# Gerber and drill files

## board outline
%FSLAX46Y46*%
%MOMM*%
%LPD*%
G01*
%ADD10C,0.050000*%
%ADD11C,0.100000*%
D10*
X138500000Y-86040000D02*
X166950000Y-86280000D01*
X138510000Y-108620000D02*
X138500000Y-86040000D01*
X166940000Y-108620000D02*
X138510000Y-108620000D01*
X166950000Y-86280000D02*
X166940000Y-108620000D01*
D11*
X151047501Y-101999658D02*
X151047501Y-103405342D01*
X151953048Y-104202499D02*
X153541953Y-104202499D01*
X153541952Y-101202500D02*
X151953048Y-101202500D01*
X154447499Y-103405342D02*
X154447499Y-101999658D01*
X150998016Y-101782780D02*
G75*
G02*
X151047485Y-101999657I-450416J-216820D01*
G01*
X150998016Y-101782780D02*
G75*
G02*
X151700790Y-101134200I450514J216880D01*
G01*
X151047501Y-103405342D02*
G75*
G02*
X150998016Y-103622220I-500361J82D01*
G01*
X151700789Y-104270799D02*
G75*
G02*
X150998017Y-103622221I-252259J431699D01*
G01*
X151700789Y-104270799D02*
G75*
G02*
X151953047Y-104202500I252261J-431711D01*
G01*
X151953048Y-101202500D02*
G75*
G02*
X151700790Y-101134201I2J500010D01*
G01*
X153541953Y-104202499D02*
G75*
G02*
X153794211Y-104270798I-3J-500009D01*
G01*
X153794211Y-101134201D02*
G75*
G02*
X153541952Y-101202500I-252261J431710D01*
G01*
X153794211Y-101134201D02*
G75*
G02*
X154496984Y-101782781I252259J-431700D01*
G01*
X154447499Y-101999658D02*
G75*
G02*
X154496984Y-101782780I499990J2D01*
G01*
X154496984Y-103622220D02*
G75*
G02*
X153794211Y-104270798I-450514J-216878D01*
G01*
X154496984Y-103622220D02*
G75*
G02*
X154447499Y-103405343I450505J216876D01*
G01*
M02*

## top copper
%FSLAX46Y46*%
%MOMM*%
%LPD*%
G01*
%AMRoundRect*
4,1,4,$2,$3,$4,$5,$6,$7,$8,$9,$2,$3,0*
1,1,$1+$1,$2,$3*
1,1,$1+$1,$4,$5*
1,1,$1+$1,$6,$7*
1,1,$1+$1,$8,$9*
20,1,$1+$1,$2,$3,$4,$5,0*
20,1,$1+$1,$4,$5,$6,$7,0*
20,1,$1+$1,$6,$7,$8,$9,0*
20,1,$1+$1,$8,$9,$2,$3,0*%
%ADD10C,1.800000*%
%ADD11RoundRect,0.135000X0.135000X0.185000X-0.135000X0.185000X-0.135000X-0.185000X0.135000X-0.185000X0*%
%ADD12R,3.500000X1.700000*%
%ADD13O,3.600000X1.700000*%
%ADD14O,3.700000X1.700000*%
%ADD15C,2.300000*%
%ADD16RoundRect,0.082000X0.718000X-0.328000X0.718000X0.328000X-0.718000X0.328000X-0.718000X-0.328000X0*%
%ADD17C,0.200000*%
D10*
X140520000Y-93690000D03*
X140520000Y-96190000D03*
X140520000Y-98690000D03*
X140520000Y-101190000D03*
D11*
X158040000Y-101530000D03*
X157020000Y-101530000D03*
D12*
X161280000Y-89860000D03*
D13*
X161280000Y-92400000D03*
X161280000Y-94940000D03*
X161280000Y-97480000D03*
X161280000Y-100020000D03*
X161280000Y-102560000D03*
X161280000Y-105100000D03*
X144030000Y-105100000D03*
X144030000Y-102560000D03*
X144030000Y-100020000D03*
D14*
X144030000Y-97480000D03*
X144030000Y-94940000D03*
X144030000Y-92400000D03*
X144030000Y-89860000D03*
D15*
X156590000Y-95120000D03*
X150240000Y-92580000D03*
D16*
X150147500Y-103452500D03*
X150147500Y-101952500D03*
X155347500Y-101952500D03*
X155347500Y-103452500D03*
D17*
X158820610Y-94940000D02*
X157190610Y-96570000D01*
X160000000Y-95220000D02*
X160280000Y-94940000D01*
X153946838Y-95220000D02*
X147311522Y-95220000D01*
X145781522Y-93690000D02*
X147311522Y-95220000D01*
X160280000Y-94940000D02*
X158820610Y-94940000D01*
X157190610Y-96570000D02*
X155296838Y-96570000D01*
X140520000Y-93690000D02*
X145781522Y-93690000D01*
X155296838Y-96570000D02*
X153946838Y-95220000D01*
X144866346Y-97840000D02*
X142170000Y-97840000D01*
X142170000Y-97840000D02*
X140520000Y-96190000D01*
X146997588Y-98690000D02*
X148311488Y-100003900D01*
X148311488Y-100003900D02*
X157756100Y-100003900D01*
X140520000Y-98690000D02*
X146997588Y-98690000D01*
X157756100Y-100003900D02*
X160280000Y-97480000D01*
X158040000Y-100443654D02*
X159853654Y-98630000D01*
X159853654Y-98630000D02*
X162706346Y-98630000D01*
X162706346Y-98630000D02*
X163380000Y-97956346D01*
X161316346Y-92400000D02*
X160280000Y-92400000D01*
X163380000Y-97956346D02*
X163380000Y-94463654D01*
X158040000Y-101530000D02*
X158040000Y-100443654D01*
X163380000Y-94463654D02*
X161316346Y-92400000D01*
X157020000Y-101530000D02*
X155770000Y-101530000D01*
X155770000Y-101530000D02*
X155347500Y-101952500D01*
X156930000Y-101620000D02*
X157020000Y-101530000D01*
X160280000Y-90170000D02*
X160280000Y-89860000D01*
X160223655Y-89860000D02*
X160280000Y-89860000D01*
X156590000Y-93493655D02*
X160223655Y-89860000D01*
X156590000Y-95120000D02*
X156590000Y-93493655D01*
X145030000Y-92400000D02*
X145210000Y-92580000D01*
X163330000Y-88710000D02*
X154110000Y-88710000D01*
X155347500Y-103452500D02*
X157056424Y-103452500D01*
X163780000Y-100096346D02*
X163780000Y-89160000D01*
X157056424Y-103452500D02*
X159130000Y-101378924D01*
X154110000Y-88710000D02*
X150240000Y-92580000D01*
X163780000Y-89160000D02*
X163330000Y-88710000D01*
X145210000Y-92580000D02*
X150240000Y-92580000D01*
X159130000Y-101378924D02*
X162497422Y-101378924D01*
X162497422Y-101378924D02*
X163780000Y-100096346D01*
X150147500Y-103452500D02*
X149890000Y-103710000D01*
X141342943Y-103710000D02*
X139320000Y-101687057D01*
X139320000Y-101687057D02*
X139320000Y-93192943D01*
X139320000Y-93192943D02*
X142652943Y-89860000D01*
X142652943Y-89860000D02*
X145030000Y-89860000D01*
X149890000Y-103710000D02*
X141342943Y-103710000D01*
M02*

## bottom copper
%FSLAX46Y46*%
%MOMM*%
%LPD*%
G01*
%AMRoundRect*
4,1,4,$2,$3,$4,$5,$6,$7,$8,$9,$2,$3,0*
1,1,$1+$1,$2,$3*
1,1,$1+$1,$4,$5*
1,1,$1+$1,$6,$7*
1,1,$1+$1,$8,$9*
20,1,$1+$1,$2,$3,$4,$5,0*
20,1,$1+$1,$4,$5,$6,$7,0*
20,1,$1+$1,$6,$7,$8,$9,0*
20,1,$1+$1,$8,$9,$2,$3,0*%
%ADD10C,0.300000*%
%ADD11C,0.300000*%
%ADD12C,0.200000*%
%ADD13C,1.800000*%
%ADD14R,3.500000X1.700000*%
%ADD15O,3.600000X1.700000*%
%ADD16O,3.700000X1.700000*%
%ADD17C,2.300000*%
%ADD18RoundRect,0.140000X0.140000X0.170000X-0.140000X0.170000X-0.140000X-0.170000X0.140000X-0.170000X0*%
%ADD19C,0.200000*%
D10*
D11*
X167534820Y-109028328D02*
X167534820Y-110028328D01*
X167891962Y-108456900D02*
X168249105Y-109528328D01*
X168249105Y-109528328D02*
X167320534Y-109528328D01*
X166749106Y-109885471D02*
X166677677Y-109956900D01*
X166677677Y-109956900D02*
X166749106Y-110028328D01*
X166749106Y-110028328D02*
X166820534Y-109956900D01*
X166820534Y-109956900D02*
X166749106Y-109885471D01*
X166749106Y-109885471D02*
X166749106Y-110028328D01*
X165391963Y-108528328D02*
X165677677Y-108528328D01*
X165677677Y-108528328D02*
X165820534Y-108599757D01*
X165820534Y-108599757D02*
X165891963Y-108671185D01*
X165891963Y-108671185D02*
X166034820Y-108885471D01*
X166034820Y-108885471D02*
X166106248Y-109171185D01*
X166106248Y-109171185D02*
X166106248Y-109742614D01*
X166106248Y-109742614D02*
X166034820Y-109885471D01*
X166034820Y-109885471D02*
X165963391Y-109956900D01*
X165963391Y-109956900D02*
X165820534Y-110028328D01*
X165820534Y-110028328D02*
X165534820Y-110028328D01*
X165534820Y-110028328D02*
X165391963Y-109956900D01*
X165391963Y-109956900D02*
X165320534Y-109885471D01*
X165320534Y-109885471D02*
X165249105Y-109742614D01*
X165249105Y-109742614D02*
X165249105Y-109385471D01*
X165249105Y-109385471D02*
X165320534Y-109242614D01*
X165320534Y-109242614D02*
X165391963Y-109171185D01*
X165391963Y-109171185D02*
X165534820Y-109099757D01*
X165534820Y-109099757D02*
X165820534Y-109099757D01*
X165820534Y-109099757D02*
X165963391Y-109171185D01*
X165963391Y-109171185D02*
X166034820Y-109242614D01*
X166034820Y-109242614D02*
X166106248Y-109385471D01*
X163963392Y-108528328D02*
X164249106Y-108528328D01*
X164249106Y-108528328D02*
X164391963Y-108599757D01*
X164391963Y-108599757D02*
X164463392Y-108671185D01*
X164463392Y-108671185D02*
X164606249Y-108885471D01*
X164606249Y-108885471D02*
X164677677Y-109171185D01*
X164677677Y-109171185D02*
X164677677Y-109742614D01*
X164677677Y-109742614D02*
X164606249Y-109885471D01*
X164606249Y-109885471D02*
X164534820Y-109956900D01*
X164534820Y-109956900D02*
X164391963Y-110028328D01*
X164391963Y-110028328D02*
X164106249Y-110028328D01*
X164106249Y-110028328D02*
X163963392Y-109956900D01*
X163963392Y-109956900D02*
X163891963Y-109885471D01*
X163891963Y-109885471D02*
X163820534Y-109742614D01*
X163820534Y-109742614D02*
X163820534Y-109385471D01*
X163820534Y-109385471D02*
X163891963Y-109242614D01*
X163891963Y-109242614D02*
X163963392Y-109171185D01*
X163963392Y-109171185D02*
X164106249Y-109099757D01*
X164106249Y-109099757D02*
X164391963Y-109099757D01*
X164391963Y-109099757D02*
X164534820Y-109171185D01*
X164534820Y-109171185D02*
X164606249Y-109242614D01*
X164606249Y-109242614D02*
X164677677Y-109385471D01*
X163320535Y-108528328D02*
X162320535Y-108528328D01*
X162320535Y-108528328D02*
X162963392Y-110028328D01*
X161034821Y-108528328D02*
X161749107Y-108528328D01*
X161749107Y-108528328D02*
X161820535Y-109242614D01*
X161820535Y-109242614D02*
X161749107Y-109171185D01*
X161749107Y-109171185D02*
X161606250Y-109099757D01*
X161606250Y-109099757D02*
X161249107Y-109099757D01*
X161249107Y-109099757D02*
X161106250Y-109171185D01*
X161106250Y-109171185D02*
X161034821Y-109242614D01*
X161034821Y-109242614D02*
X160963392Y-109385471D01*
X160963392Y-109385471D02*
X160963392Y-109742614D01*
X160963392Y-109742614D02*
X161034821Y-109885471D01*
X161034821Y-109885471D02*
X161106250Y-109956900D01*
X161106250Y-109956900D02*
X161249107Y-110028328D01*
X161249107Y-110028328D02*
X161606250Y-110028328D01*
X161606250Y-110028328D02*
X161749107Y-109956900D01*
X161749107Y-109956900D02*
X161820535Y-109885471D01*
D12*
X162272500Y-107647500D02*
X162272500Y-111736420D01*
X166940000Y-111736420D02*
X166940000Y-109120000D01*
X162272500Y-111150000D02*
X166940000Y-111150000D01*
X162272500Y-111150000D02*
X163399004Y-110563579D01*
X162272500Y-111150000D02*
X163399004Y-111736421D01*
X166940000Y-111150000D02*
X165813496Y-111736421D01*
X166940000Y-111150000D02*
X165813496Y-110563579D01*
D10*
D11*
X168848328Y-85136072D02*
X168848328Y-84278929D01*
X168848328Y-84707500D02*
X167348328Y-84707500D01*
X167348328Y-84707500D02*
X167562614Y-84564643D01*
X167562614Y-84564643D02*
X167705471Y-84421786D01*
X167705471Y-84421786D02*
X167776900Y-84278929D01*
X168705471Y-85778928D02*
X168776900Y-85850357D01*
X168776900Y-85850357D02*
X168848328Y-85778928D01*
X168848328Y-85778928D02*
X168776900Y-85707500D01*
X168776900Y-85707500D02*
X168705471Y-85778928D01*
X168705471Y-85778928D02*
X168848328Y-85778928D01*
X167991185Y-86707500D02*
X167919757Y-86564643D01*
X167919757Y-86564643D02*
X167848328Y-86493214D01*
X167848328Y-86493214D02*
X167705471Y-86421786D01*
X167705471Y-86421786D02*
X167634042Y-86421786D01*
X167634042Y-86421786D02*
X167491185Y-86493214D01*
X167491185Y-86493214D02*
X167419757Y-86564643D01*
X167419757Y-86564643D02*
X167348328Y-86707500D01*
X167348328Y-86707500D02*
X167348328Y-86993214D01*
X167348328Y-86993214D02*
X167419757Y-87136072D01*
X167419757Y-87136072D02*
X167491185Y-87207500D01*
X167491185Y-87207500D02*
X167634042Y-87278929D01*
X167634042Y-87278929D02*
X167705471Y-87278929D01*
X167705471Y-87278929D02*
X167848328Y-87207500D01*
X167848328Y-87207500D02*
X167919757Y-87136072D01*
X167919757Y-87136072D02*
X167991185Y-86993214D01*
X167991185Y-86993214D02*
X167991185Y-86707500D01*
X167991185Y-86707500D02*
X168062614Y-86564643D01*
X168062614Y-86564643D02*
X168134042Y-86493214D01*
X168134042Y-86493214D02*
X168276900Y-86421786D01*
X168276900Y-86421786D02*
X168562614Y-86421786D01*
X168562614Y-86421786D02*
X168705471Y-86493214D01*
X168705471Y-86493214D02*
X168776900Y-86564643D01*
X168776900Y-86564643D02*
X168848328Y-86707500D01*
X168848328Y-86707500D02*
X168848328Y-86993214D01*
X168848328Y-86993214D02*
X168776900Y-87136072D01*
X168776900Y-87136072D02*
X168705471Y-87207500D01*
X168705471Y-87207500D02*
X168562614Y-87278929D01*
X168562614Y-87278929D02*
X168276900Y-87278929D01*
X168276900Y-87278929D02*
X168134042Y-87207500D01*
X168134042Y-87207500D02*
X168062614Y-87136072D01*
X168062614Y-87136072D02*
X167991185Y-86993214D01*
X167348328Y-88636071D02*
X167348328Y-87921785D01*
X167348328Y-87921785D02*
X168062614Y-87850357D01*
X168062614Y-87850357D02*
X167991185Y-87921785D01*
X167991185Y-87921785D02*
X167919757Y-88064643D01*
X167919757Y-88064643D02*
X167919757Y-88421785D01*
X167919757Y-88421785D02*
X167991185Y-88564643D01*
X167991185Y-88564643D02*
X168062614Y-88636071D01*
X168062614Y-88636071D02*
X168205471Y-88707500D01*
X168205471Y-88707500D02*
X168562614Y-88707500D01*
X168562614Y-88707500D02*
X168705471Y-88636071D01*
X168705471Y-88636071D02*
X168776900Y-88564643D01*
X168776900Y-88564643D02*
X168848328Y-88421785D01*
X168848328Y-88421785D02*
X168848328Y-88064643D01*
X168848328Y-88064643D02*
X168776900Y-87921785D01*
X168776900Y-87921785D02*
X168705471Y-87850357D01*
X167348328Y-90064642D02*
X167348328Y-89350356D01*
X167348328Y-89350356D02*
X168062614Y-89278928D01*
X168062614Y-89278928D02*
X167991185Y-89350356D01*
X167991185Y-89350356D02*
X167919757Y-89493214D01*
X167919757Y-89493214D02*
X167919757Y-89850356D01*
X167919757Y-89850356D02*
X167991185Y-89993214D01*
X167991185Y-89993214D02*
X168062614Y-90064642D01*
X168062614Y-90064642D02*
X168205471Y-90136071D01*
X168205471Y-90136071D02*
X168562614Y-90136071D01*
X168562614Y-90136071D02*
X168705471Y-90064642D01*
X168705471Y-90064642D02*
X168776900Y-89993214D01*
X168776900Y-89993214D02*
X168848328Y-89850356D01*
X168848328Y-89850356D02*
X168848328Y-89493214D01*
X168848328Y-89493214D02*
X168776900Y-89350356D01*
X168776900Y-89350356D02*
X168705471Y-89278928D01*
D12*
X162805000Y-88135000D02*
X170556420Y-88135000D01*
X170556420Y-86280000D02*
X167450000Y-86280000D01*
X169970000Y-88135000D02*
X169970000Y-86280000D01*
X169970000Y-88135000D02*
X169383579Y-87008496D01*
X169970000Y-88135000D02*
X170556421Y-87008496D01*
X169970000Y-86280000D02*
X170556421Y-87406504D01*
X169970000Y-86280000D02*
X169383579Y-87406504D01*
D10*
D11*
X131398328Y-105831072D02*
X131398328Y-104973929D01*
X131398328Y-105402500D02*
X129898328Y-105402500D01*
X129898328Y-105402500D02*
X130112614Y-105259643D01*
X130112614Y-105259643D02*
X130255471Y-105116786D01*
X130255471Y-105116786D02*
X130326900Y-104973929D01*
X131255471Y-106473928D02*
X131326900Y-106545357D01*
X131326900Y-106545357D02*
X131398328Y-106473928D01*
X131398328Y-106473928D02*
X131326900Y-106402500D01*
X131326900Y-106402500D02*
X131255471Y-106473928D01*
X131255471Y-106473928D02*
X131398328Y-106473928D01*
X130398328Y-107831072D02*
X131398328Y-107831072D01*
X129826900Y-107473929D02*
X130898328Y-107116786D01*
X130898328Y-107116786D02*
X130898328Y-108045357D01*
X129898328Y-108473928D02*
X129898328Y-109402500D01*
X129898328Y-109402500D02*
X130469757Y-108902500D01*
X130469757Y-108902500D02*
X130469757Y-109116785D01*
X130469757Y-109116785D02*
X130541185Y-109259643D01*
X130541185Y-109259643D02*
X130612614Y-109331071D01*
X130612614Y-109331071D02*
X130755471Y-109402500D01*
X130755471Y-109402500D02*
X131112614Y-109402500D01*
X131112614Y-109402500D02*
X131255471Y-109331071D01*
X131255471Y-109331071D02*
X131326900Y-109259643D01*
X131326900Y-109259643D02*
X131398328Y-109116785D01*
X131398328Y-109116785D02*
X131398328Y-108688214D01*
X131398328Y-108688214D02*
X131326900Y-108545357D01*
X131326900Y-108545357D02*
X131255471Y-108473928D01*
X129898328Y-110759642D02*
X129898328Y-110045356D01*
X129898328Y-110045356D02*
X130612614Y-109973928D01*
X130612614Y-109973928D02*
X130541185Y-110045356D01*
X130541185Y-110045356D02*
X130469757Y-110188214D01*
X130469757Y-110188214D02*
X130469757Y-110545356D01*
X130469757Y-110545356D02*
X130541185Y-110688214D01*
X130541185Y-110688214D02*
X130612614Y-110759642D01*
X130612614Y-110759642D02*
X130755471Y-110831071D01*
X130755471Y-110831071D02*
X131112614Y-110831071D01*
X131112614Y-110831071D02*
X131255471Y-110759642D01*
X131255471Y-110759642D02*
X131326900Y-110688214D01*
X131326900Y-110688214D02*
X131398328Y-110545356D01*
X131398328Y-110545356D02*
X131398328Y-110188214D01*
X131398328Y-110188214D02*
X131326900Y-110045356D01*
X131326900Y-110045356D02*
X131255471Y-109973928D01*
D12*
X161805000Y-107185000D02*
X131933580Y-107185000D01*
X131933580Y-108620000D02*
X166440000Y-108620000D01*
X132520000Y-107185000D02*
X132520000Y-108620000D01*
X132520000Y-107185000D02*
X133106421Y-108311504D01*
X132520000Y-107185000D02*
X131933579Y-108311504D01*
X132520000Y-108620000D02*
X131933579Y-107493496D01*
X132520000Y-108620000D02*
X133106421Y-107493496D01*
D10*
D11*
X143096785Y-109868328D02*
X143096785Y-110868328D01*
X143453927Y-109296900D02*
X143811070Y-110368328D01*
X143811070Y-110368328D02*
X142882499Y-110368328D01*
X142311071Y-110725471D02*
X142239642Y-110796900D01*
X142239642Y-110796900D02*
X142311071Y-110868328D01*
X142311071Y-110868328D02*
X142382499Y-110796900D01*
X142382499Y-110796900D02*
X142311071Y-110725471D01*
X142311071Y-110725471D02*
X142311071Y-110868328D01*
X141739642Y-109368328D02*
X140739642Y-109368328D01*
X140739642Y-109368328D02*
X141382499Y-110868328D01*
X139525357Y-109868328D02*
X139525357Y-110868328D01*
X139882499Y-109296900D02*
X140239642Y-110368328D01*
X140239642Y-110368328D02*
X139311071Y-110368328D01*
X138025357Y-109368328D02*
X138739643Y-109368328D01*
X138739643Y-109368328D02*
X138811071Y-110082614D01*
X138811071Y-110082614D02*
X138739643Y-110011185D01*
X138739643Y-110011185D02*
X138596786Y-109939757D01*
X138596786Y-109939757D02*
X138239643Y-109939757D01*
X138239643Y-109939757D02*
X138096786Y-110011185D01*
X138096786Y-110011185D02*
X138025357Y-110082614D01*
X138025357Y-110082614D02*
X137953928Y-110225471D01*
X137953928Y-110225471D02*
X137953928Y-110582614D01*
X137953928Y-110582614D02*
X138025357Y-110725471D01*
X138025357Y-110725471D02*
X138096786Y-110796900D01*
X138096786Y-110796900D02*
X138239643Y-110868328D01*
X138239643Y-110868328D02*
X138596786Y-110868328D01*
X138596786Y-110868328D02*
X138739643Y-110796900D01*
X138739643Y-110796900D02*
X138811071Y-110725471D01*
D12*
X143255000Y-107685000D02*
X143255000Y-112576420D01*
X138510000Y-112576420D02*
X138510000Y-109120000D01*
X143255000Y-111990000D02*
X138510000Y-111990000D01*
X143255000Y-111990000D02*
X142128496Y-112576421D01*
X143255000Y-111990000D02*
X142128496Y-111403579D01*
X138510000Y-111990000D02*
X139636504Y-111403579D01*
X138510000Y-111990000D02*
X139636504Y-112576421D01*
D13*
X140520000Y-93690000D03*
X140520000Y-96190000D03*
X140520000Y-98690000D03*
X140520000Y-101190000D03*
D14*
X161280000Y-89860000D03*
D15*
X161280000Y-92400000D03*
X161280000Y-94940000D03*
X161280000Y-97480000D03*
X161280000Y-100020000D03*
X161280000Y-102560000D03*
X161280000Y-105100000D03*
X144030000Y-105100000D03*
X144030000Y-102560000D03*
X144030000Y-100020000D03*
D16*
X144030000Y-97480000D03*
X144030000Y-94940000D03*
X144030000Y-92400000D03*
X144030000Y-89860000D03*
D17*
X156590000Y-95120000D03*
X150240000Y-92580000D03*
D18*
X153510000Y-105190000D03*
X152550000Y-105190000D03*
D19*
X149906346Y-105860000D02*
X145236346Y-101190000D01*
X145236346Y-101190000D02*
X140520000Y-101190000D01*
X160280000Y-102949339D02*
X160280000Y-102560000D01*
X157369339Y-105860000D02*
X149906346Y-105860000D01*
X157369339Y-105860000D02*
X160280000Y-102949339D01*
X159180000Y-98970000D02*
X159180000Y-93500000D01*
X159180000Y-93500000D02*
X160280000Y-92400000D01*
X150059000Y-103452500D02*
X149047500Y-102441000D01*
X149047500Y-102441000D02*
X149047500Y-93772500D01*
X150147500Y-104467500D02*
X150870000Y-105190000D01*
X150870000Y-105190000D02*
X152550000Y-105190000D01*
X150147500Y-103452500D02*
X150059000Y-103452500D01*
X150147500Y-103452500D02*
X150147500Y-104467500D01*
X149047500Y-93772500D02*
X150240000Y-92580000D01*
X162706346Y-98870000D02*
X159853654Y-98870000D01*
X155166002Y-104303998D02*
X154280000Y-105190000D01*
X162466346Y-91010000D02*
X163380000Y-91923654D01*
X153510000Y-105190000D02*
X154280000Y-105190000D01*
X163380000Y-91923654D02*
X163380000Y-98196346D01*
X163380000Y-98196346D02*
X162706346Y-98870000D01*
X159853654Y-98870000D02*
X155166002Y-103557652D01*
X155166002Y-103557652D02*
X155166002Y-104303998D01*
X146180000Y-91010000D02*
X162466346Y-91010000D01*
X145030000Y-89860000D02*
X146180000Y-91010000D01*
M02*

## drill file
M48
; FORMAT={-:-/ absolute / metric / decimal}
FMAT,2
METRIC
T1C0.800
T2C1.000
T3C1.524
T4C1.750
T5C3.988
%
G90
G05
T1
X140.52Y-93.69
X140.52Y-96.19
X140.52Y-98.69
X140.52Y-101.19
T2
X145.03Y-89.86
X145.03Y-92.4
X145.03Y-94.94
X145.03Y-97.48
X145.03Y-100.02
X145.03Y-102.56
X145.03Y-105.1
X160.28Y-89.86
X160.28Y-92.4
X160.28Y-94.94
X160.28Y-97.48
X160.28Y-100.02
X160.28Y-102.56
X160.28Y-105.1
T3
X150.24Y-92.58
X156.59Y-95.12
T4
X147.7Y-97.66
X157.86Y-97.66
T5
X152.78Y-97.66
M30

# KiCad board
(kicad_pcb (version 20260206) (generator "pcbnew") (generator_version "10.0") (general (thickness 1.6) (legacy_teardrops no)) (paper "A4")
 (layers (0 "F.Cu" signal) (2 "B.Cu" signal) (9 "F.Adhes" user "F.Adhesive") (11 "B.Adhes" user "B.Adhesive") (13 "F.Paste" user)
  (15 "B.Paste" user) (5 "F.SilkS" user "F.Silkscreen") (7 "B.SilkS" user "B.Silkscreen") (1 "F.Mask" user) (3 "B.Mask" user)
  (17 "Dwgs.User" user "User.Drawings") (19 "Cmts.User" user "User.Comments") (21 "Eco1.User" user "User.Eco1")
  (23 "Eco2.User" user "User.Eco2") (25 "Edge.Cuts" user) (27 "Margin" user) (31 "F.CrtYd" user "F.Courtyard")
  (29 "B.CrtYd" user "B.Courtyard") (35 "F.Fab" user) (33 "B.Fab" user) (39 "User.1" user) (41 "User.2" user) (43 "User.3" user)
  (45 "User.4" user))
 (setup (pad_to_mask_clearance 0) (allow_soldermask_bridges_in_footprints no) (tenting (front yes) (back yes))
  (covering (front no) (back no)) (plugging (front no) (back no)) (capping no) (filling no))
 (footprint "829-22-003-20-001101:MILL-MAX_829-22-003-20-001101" (layer "F.Cu") (at 137.32 85.84)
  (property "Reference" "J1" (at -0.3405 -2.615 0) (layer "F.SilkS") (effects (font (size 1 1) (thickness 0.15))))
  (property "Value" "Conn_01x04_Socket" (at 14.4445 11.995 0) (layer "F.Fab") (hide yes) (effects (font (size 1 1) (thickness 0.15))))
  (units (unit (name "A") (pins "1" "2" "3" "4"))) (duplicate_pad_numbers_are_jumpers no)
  (pad "1" thru_hole circle (at 3.2 7.85 270) (size 1.8 1.8) (drill 0.8) (layers "*.Cu" "*.Mask") (remove_unused_layers no)
   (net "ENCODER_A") (solder_mask_margin 0.102))
  (pad "2" thru_hole circle (at 3.2 10.35 270) (size 1.8 1.8) (drill 0.8) (layers "*.Cu" "*.Mask") (remove_unused_layers no) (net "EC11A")
   (solder_mask_margin 0.102))
  (pad "3" thru_hole circle (at 3.2 12.85 270) (size 1.8 1.8) (drill 0.8) (layers "*.Cu" "*.Mask") (remove_unused_layers no)
   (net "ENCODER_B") (solder_mask_margin 0.102))
  (pad "4" thru_hole circle (at 3.2 15.35 270) (size 1.8 1.8) (drill 0.8) (layers "*.Cu" "*.Mask") (remove_unused_layers no) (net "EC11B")
   (solder_mask_margin 0.102)))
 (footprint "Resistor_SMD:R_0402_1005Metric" (layer "F.Cu") (at 157.53 101.53 180)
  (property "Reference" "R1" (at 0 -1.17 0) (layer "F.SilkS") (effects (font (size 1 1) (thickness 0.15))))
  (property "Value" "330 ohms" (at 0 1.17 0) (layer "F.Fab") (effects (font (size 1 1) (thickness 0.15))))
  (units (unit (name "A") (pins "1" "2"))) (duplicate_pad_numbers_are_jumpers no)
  (pad "1" smd roundrect (at -0.51 0 180) (size 0.54 0.64) (layers "F.Cu" "F.Mask" "F.Paste") (roundrect_rratio 0.25) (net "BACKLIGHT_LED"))
  (pad "2" smd roundrect (at 0.51 0 180) (size 0.54 0.64) (layers "F.Cu" "F.Mask" "F.Paste") (roundrect_rratio 0.25) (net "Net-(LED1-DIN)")))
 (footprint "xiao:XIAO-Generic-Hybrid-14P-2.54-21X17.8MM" (layer "B.Cu") (at 152.655 97.48 180)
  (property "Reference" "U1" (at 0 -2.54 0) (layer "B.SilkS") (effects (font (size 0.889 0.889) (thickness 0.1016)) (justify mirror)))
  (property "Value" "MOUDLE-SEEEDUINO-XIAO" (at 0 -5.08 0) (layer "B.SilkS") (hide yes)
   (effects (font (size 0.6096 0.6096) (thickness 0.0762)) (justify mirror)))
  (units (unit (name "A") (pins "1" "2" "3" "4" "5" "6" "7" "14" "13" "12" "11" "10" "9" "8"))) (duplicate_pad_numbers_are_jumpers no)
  (pad "1" thru_hole rect (at -7.625 7.62 180) (size 3.5 1.7) (drill 1 (offset -1 0)) (layers "*.Cu" "*.Mask") (remove_unused_layers no)
   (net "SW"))
  (pad "2" thru_hole oval (at -7.625 5.08 180) (size 3.6 1.7) (drill 1 (offset -1 0)) (layers "*.Cu" "*.Mask") (remove_unused_layers no)
   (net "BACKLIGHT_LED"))
  (pad "3" thru_hole oval (at -7.625 2.54 180) (size 3.6 1.7) (drill 1 (offset -1 0)) (layers "*.Cu" "*.Mask") (remove_unused_layers no)
   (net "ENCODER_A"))
  (pad "4" thru_hole oval (at -7.625 0 180) (size 3.6 1.7) (drill 1 (offset -1 0)) (layers "*.Cu" "*.Mask") (remove_unused_layers no)
   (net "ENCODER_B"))
  (pad "5" thru_hole oval (at -7.625 -2.54 180) (size 3.6 1.7) (drill 1 (offset -1 0)) (layers "*.Cu" "*.Mask") (remove_unused_layers no)
   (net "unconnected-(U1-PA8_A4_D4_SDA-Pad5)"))
  (pad "6" thru_hole oval (at -7.625 -5.08) (size 3.6 1.7) (drill 1 (offset 1 0)) (layers "*.Cu" "*.Mask") (remove_unused_layers no)
   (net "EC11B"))
  (pad "7" thru_hole oval (at -7.625 -7.62 180) (size 3.6 1.7) (drill 1 (offset -1 0)) (layers "*.Cu" "*.Mask") (remove_unused_layers no)
   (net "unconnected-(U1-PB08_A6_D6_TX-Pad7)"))
  (pad "8" thru_hole oval (at 7.625 -7.62 180) (size 3.6 1.7) (drill 1 (offset 1 0)) (layers "*.Cu" "*.Mask") (remove_unused_layers no)
   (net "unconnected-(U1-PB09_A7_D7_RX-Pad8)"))
  (pad "9" thru_hole oval (at 7.625 -5.08 180) (size 3.6 1.7) (drill 1 (offset 1 0)) (layers "*.Cu" "*.Mask") (remove_unused_layers no)
   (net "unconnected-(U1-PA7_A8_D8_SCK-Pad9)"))
  (pad "10" thru_hole oval (at 7.625 -2.54 180) (size 3.6 1.7) (drill 1 (offset 1 0)) (layers "*.Cu" "*.Mask") (remove_unused_layers no)
   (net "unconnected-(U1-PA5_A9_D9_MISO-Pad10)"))
  (pad "11" thru_hole oval (at 7.625 0 180) (size 3.7 1.7) (drill 1 (offset 1 0)) (layers "*.Cu" "*.Mask") (remove_unused_layers no)
   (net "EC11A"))
  (pad "12" thru_hole oval (at 7.625 2.54 180) (size 3.7 1.7) (drill 1 (offset 1 0)) (layers "*.Cu" "*.Mask") (remove_unused_layers no)
   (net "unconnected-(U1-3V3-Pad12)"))
  (pad "13" thru_hole oval (at 7.625 5.08 180) (size 3.7 1.7) (drill 1 (offset 1 0)) (layers "*.Cu" "*.Mask") (remove_unused_layers no)
   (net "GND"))
  (pad "14" thru_hole oval (at 7.625 7.62 180) (size 3.7 1.7) (drill 1 (offset 1 0)) (layers "*.Cu" "*.Mask") (remove_unused_layers no)
   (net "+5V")))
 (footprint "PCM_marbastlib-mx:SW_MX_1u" (layer "B.Cu") (at 152.78 97.66 180)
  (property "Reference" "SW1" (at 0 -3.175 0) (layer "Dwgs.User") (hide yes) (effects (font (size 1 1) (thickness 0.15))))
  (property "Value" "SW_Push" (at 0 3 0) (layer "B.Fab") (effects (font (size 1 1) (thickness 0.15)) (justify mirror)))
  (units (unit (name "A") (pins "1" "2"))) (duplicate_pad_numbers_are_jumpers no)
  (pad "" np_thru_hole circle (at -5.08 0 180) (size 1.75 1.75) (drill 1.75) (layers "*.Cu" "*.Mask"))
  (pad "" np_thru_hole circle (at 0 0 180) (size 3.9878 3.9878) (drill 3.9878) (layers "*.Cu" "*.Mask"))
  (pad "" np_thru_hole circle (at 5.08 0 180) (size 1.75 1.75) (drill 1.75) (layers "*.Cu" "*.Mask"))
  (pad "1" thru_hole circle (at -3.81 2.54 180) (size 2.3 2.3) (drill 1.524) (layers "*.Cu" "F.Mask") (remove_unused_layers no) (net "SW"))
  (pad "2" thru_hole circle (at 2.54 5.08 180) (size 2.3 2.3) (drill 1.524) (layers "*.Cu" "F.Mask") (remove_unused_layers no) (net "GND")))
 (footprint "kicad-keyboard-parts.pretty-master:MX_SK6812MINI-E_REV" (layer "B.Cu") (at 152.7475 97.6225 180)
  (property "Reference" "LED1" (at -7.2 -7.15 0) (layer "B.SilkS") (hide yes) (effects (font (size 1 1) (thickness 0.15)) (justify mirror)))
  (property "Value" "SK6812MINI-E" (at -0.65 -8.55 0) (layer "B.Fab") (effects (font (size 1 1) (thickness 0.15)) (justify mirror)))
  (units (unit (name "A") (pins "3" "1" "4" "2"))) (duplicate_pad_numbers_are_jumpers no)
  (fp_line (start 1.699999 -4.377158) (end 1.699999 -5.782842) (stroke (width 0.1) (type solid)) (layer "Edge.Cuts"))
  (fp_line (start 0.794452 -6.579999) (end -0.794453 -6.579999) (stroke (width 0.1) (type solid)) (layer "Edge.Cuts"))
  (fp_line (start -0.794452 -3.58) (end 0.794452 -3.58) (stroke (width 0.1) (type solid)) (layer "Edge.Cuts"))
  (fp_line (start -1.699999 -5.782842) (end -1.699999 -4.377158) (stroke (width 0.1) (type solid)) (layer "Edge.Cuts"))
  (fp_arc (start 1.749484 -4.16028) (mid 1.712526 -4.265931) (end 1.699999 -4.377157) (stroke (width 0.1) (type solid)) (layer "Edge.Cuts"))
  (fp_arc (start 1.749484 -4.16028) (mid 1.638072 -3.575963) (end 1.046711 -3.511703) (stroke (width 0.1) (type solid)) (layer "Edge.Cuts"))
  (fp_arc (start 1.699999 -5.782842) (mid 1.712536 -5.894065) (end 1.749484 -5.99972) (stroke (width 0.1) (type solid)) (layer "Edge.Cuts"))
  (fp_arc (start 1.046711 -6.648299) (mid 1.638071 -6.584036) (end 1.749484 -5.99972) (stroke (width 0.1) (type solid)) (layer "Edge.Cuts"))
  (fp_arc (start 1.046711 -6.648299) (mid 0.925123 -6.597377) (end 0.794453 -6.58) (stroke (width 0.1) (type solid)) (layer "Edge.Cuts"))
  (fp_arc (start 0.794452 -3.58) (mid 0.925122 -3.562623) (end 1.04671 -3.511701) (stroke (width 0.1) (type solid)) (layer "Edge.Cuts"))
  (fp_arc (start -0.794453 -6.579999) (mid -0.925123 -6.597376) (end -1.046711 -6.648298) (stroke (width 0.1) (type solid))
   (layer "Edge.Cuts"))
  (fp_arc (start -1.046711 -3.511701) (mid -0.925123 -3.562623) (end -0.794452 -3.58) (stroke (width 0.1) (type solid)) (layer "Edge.Cuts"))
  (fp_arc (start -1.046711 -3.511701) (mid -1.638072 -3.575965) (end -1.749484 -4.160281) (stroke (width 0.1) (type solid))
   (layer "Edge.Cuts"))
  (fp_arc (start -1.699999 -4.377158) (mid -1.712527 -4.265932) (end -1.749484 -4.16028) (stroke (width 0.1) (type solid))
   (layer "Edge.Cuts"))
  (fp_arc (start -1.749484 -5.99972) (mid -1.638071 -6.584035) (end -1.046711 -6.648298) (stroke (width 0.1) (type solid))
   (layer "Edge.Cuts"))
  (fp_arc (start -1.749484 -5.99972) (mid -1.712527 -5.894068) (end -1.699999 -5.782843) (stroke (width 0.1) (type solid))
   (layer "Edge.Cuts"))
  (pad "1" smd roundrect (at 2.6 -5.83 90) (size 0.82 1.6) (layers "F.Cu" "F.Mask" "F.Paste") (roundrect_rratio 0.1) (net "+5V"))
  (pad "2" smd roundrect (at 2.6 -4.33 90) (size 0.82 1.6) (layers "F.Cu" "F.Mask" "F.Paste") (roundrect_rratio 0.1)
   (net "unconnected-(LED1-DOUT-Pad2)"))
  (pad "3" smd roundrect (at -2.6 -4.33 90) (size 0.82 1.6) (layers "F.Cu" "F.Mask" "F.Paste") (roundrect_rratio 0.1) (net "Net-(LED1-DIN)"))
  (pad "4" smd roundrect (at -2.6 -5.83 90) (size 0.82 1.6) (layers "F.Cu" "F.Mask" "F.Paste") (roundrect_rratio 0.1) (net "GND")))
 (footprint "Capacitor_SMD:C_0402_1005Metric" (layer "B.Cu") (at 153.03 105.19 180)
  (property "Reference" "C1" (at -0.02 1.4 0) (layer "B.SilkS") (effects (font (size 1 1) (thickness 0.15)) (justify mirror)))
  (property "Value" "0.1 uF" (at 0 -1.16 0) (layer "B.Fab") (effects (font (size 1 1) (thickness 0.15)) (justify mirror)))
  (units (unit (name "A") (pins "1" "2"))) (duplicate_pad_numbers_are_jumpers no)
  (pad "1" smd roundrect (at -0.48 0 180) (size 0.56 0.62) (layers "B.Cu" "B.Mask" "B.Paste") (roundrect_rratio 0.25) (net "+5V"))
  (pad "2" smd roundrect (at 0.48 0 180) (size 0.56 0.62) (layers "B.Cu" "B.Mask" "B.Paste") (roundrect_rratio 0.25) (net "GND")))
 (gr_line (start 138.5 86.04) (end 166.95 86.28) (stroke (width 0.05) (type default)) (layer "Edge.Cuts"))
 (gr_line (start 138.51 108.62) (end 138.5 86.04) (stroke (width 0.05) (type default)) (layer "Edge.Cuts"))
 (gr_line (start 166.94 108.62) (end 138.51 108.62) (stroke (width 0.05) (type default)) (layer "Edge.Cuts"))
 (gr_line (start 166.95 86.28) (end 166.94 108.62) (stroke (width 0.05) (type default)) (layer "Edge.Cuts"))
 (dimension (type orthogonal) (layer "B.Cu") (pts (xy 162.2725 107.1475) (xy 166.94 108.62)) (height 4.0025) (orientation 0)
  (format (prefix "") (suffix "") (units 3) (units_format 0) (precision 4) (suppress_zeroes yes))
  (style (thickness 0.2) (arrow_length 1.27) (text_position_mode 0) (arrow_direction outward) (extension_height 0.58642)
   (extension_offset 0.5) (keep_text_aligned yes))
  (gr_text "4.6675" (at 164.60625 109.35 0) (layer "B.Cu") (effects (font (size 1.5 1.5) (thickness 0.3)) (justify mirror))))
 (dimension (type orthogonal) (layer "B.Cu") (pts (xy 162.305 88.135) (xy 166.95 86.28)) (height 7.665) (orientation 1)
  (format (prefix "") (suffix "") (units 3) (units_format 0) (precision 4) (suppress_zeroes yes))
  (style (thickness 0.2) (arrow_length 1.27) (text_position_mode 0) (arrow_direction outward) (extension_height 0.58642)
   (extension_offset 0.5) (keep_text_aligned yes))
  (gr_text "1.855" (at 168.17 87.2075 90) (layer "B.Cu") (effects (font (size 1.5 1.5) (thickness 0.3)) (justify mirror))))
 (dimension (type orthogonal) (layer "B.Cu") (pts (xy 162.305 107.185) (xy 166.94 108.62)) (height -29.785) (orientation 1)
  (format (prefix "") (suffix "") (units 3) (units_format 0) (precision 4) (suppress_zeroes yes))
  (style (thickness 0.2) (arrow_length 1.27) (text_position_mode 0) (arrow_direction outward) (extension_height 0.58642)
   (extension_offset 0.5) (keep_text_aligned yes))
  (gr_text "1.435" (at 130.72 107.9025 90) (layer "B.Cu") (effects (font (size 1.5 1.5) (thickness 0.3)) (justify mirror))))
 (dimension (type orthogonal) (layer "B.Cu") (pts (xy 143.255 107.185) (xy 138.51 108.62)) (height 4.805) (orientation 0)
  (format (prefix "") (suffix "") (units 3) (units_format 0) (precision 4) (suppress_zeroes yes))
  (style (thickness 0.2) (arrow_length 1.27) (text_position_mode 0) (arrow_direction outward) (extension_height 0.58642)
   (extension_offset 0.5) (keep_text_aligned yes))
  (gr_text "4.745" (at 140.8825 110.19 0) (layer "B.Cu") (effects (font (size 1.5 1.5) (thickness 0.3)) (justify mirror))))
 (segment (start 158.82061 94.94) (end 157.19061 96.57) (width 0.2) (layer "F.Cu") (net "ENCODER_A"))
 (segment (start 160 95.22) (end 160.28 94.94) (width 0.2) (layer "F.Cu") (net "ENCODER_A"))
 (segment (start 153.946838 95.22) (end 147.311522 95.22) (width 0.2) (layer "F.Cu") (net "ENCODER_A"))
 (segment (start 145.781522 93.69) (end 147.311522 95.22) (width 0.2) (layer "F.Cu") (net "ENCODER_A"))
 (segment (start 160.28 94.94) (end 158.82061 94.94) (width 0.2) (layer "F.Cu") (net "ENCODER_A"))
 (segment (start 157.19061 96.57) (end 155.296838 96.57) (width 0.2) (layer "F.Cu") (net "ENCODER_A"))
 (segment (start 140.52 93.69) (end 145.781522 93.69) (width 0.2) (layer "F.Cu") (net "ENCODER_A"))
 (segment (start 155.296838 96.57) (end 153.946838 95.22) (width 0.2) (layer "F.Cu") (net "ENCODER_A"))
 (segment (start 144.866346 97.84) (end 142.17 97.84) (width 0.2) (layer "F.Cu") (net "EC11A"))
 (segment (start 142.17 97.84) (end 140.52 96.19) (width 0.2) (layer "F.Cu") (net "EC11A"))
 (segment (start 146.997588 98.69) (end 148.311488 100.0039) (width 0.2) (layer "F.Cu") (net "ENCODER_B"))
 (segment (start 148.311488 100.0039) (end 157.7561 100.0039) (width 0.2) (layer "F.Cu") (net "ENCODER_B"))
 (segment (start 140.52 98.69) (end 146.997588 98.69) (width 0.2) (layer "F.Cu") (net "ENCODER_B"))
 (segment (start 157.7561 100.0039) (end 160.28 97.48) (width 0.2) (layer "F.Cu") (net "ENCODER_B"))
 (segment (start 149.906346 105.86) (end 145.236346 101.19) (width 0.2) (layer "B.Cu") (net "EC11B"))
 (segment (start 145.236346 101.19) (end 140.52 101.19) (width 0.2) (layer "B.Cu") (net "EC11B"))
 (segment (start 160.28 102.949339) (end 160.28 102.56) (width 0.2) (layer "B.Cu") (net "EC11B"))
 (segment (start 157.369339 105.86) (end 149.906346 105.86) (width 0.2) (layer "B.Cu") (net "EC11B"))
 (segment (start 157.369339 105.86) (end 160.28 102.949339) (width 0.2) (layer "B.Cu") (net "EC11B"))
 (segment (start 158.04 100.443654) (end 159.853654 98.63) (width 0.2) (layer "F.Cu") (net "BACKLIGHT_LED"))
 (segment (start 159.853654 98.63) (end 162.706346 98.63) (width 0.2) (layer "F.Cu") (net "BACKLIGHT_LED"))
 (segment (start 162.706346 98.63) (end 163.38 97.956346) (width 0.2) (layer "F.Cu") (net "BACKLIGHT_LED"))
 (segment (start 161.316346 92.4) (end 160.28 92.4) (width 0.2) (layer "F.Cu") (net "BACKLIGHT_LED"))
 (segment (start 163.38 97.956346) (end 163.38 94.463654) (width 0.2) (layer "F.Cu") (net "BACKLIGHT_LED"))
 (segment (start 158.04 101.53) (end 158.04 100.443654) (width 0.2) (layer "F.Cu") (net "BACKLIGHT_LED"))
 (segment (start 163.38 94.463654) (end 161.316346 92.4) (width 0.2) (layer "F.Cu") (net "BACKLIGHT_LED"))
 (segment (start 159.18 98.97) (end 159.18 93.5) (width 0.2) (layer "B.Cu") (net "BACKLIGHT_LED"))
 (segment (start 159.18 93.5) (end 160.28 92.4) (width 0.2) (layer "B.Cu") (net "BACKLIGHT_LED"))
 (segment (start 157.02 101.53) (end 155.77 101.53) (width 0.2) (layer "F.Cu") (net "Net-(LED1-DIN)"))
 (segment (start 155.77 101.53) (end 155.3475 101.9525) (width 0.2) (layer "F.Cu") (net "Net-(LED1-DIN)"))
 (segment (start 156.93 101.62) (end 157.02 101.53) (width 0.2) (layer "F.Cu") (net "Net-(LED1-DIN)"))
 (segment (start 160.28 90.17) (end 160.28 89.86) (width 0.2) (layer "F.Cu") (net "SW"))
 (segment (start 160.223655 89.86) (end 160.28 89.86) (width 0.2) (layer "F.Cu") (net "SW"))
 (segment (start 156.59 93.493655) (end 160.223655 89.86) (width 0.2) (layer "F.Cu") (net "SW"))
 (segment (start 156.59 95.12) (end 156.59 93.493655) (width 0.2) (layer "F.Cu") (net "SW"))
 (segment (start 145.03 92.4) (end 145.21 92.58) (width 0.2) (layer "F.Cu") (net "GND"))
 (segment (start 163.33 88.71) (end 154.11 88.71) (width 0.2) (layer "F.Cu") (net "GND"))
 (segment (start 155.3475 103.4525) (end 157.056424 103.4525) (width 0.2) (layer "F.Cu") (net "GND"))
 (segment (start 163.78 100.096346) (end 163.78 89.16) (width 0.2) (layer "F.Cu") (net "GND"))
 (segment (start 157.056424 103.4525) (end 159.13 101.378924) (width 0.2) (layer "F.Cu") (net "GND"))
 (segment (start 154.11 88.71) (end 150.24 92.58) (width 0.2) (layer "F.Cu") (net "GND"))
 (segment (start 163.78 89.16) (end 163.33 88.71) (width 0.2) (layer "F.Cu") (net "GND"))
 (segment (start 145.21 92.58) (end 150.24 92.58) (width 0.2) (layer "F.Cu") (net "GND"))
 (segment (start 159.13 101.378924) (end 162.497422 101.378924) (width 0.2) (layer "F.Cu") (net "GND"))
 (segment (start 162.497422 101.378924) (end 163.78 100.096346) (width 0.2) (layer "F.Cu") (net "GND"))
 (segment (start 150.059 103.4525) (end 149.0475 102.441) (width 0.2) (layer "B.Cu") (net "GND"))
 (segment (start 149.0475 102.441) (end 149.0475 93.7725) (width 0.2) (layer "B.Cu") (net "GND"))
 (segment (start 150.1475 104.4675) (end 150.87 105.19) (width 0.2) (layer "B.Cu") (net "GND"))
 (segment (start 150.87 105.19) (end 152.55 105.19) (width 0.2) (layer "B.Cu") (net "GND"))
 (segment (start 150.1475 103.4525) (end 150.059 103.4525) (width 0.2) (layer "B.Cu") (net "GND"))
 (segment (start 150.1475 103.4525) (end 150.1475 104.4675) (width 0.2) (layer "B.Cu") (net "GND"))
 (segment (start 149.0475 93.7725) (end 150.24 92.58) (width 0.2) (layer "B.Cu") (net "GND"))
 (segment (start 150.1475 103.4525) (end 149.89 103.71) (width 0.2) (layer "F.Cu") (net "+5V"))
 (segment (start 141.342943 103.71) (end 139.32 101.687057) (width 0.2) (layer "F.Cu") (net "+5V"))
 (segment (start 139.32 101.687057) (end 139.32 93.192943) (width 0.2) (layer "F.Cu") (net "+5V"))
 (segment (start 139.32 93.192943) (end 142.652943 89.86) (width 0.2) (layer "F.Cu") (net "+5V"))
 (segment (start 142.652943 89.86) (end 145.03 89.86) (width 0.2) (layer "F.Cu") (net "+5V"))
 (segment (start 149.89 103.71) (end 141.342943 103.71) (width 0.2) (layer "F.Cu") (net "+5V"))
 (segment (start 162.706346 98.87) (end 159.853654 98.87) (width 0.2) (layer "B.Cu") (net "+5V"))
 (segment (start 155.166002 104.303998) (end 154.28 105.19) (width 0.2) (layer "B.Cu") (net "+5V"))
 (segment (start 162.466346 91.01) (end 163.38 91.923654) (width 0.2) (layer "B.Cu") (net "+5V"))
 (segment (start 153.51 105.19) (end 154.28 105.19) (width 0.2) (layer "B.Cu") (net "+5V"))
 (segment (start 163.38 91.923654) (end 163.38 98.196346) (width 0.2) (layer "B.Cu") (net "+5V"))
 (segment (start 163.38 98.196346) (end 162.706346 98.87) (width 0.2) (layer "B.Cu") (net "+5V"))
 (segment (start 159.853654 98.87) (end 155.166002 103.557652) (width 0.2) (layer "B.Cu") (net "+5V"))
 (segment (start 155.166002 103.557652) (end 155.166002 104.303998) (width 0.2) (layer "B.Cu") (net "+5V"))
 (segment (start 146.18 91.01) (end 162.466346 91.01) (width 0.2) (layer "B.Cu") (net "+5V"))
 (segment (start 145.03 89.86) (end 146.18 91.01) (width 0.2) (layer "B.Cu") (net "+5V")))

